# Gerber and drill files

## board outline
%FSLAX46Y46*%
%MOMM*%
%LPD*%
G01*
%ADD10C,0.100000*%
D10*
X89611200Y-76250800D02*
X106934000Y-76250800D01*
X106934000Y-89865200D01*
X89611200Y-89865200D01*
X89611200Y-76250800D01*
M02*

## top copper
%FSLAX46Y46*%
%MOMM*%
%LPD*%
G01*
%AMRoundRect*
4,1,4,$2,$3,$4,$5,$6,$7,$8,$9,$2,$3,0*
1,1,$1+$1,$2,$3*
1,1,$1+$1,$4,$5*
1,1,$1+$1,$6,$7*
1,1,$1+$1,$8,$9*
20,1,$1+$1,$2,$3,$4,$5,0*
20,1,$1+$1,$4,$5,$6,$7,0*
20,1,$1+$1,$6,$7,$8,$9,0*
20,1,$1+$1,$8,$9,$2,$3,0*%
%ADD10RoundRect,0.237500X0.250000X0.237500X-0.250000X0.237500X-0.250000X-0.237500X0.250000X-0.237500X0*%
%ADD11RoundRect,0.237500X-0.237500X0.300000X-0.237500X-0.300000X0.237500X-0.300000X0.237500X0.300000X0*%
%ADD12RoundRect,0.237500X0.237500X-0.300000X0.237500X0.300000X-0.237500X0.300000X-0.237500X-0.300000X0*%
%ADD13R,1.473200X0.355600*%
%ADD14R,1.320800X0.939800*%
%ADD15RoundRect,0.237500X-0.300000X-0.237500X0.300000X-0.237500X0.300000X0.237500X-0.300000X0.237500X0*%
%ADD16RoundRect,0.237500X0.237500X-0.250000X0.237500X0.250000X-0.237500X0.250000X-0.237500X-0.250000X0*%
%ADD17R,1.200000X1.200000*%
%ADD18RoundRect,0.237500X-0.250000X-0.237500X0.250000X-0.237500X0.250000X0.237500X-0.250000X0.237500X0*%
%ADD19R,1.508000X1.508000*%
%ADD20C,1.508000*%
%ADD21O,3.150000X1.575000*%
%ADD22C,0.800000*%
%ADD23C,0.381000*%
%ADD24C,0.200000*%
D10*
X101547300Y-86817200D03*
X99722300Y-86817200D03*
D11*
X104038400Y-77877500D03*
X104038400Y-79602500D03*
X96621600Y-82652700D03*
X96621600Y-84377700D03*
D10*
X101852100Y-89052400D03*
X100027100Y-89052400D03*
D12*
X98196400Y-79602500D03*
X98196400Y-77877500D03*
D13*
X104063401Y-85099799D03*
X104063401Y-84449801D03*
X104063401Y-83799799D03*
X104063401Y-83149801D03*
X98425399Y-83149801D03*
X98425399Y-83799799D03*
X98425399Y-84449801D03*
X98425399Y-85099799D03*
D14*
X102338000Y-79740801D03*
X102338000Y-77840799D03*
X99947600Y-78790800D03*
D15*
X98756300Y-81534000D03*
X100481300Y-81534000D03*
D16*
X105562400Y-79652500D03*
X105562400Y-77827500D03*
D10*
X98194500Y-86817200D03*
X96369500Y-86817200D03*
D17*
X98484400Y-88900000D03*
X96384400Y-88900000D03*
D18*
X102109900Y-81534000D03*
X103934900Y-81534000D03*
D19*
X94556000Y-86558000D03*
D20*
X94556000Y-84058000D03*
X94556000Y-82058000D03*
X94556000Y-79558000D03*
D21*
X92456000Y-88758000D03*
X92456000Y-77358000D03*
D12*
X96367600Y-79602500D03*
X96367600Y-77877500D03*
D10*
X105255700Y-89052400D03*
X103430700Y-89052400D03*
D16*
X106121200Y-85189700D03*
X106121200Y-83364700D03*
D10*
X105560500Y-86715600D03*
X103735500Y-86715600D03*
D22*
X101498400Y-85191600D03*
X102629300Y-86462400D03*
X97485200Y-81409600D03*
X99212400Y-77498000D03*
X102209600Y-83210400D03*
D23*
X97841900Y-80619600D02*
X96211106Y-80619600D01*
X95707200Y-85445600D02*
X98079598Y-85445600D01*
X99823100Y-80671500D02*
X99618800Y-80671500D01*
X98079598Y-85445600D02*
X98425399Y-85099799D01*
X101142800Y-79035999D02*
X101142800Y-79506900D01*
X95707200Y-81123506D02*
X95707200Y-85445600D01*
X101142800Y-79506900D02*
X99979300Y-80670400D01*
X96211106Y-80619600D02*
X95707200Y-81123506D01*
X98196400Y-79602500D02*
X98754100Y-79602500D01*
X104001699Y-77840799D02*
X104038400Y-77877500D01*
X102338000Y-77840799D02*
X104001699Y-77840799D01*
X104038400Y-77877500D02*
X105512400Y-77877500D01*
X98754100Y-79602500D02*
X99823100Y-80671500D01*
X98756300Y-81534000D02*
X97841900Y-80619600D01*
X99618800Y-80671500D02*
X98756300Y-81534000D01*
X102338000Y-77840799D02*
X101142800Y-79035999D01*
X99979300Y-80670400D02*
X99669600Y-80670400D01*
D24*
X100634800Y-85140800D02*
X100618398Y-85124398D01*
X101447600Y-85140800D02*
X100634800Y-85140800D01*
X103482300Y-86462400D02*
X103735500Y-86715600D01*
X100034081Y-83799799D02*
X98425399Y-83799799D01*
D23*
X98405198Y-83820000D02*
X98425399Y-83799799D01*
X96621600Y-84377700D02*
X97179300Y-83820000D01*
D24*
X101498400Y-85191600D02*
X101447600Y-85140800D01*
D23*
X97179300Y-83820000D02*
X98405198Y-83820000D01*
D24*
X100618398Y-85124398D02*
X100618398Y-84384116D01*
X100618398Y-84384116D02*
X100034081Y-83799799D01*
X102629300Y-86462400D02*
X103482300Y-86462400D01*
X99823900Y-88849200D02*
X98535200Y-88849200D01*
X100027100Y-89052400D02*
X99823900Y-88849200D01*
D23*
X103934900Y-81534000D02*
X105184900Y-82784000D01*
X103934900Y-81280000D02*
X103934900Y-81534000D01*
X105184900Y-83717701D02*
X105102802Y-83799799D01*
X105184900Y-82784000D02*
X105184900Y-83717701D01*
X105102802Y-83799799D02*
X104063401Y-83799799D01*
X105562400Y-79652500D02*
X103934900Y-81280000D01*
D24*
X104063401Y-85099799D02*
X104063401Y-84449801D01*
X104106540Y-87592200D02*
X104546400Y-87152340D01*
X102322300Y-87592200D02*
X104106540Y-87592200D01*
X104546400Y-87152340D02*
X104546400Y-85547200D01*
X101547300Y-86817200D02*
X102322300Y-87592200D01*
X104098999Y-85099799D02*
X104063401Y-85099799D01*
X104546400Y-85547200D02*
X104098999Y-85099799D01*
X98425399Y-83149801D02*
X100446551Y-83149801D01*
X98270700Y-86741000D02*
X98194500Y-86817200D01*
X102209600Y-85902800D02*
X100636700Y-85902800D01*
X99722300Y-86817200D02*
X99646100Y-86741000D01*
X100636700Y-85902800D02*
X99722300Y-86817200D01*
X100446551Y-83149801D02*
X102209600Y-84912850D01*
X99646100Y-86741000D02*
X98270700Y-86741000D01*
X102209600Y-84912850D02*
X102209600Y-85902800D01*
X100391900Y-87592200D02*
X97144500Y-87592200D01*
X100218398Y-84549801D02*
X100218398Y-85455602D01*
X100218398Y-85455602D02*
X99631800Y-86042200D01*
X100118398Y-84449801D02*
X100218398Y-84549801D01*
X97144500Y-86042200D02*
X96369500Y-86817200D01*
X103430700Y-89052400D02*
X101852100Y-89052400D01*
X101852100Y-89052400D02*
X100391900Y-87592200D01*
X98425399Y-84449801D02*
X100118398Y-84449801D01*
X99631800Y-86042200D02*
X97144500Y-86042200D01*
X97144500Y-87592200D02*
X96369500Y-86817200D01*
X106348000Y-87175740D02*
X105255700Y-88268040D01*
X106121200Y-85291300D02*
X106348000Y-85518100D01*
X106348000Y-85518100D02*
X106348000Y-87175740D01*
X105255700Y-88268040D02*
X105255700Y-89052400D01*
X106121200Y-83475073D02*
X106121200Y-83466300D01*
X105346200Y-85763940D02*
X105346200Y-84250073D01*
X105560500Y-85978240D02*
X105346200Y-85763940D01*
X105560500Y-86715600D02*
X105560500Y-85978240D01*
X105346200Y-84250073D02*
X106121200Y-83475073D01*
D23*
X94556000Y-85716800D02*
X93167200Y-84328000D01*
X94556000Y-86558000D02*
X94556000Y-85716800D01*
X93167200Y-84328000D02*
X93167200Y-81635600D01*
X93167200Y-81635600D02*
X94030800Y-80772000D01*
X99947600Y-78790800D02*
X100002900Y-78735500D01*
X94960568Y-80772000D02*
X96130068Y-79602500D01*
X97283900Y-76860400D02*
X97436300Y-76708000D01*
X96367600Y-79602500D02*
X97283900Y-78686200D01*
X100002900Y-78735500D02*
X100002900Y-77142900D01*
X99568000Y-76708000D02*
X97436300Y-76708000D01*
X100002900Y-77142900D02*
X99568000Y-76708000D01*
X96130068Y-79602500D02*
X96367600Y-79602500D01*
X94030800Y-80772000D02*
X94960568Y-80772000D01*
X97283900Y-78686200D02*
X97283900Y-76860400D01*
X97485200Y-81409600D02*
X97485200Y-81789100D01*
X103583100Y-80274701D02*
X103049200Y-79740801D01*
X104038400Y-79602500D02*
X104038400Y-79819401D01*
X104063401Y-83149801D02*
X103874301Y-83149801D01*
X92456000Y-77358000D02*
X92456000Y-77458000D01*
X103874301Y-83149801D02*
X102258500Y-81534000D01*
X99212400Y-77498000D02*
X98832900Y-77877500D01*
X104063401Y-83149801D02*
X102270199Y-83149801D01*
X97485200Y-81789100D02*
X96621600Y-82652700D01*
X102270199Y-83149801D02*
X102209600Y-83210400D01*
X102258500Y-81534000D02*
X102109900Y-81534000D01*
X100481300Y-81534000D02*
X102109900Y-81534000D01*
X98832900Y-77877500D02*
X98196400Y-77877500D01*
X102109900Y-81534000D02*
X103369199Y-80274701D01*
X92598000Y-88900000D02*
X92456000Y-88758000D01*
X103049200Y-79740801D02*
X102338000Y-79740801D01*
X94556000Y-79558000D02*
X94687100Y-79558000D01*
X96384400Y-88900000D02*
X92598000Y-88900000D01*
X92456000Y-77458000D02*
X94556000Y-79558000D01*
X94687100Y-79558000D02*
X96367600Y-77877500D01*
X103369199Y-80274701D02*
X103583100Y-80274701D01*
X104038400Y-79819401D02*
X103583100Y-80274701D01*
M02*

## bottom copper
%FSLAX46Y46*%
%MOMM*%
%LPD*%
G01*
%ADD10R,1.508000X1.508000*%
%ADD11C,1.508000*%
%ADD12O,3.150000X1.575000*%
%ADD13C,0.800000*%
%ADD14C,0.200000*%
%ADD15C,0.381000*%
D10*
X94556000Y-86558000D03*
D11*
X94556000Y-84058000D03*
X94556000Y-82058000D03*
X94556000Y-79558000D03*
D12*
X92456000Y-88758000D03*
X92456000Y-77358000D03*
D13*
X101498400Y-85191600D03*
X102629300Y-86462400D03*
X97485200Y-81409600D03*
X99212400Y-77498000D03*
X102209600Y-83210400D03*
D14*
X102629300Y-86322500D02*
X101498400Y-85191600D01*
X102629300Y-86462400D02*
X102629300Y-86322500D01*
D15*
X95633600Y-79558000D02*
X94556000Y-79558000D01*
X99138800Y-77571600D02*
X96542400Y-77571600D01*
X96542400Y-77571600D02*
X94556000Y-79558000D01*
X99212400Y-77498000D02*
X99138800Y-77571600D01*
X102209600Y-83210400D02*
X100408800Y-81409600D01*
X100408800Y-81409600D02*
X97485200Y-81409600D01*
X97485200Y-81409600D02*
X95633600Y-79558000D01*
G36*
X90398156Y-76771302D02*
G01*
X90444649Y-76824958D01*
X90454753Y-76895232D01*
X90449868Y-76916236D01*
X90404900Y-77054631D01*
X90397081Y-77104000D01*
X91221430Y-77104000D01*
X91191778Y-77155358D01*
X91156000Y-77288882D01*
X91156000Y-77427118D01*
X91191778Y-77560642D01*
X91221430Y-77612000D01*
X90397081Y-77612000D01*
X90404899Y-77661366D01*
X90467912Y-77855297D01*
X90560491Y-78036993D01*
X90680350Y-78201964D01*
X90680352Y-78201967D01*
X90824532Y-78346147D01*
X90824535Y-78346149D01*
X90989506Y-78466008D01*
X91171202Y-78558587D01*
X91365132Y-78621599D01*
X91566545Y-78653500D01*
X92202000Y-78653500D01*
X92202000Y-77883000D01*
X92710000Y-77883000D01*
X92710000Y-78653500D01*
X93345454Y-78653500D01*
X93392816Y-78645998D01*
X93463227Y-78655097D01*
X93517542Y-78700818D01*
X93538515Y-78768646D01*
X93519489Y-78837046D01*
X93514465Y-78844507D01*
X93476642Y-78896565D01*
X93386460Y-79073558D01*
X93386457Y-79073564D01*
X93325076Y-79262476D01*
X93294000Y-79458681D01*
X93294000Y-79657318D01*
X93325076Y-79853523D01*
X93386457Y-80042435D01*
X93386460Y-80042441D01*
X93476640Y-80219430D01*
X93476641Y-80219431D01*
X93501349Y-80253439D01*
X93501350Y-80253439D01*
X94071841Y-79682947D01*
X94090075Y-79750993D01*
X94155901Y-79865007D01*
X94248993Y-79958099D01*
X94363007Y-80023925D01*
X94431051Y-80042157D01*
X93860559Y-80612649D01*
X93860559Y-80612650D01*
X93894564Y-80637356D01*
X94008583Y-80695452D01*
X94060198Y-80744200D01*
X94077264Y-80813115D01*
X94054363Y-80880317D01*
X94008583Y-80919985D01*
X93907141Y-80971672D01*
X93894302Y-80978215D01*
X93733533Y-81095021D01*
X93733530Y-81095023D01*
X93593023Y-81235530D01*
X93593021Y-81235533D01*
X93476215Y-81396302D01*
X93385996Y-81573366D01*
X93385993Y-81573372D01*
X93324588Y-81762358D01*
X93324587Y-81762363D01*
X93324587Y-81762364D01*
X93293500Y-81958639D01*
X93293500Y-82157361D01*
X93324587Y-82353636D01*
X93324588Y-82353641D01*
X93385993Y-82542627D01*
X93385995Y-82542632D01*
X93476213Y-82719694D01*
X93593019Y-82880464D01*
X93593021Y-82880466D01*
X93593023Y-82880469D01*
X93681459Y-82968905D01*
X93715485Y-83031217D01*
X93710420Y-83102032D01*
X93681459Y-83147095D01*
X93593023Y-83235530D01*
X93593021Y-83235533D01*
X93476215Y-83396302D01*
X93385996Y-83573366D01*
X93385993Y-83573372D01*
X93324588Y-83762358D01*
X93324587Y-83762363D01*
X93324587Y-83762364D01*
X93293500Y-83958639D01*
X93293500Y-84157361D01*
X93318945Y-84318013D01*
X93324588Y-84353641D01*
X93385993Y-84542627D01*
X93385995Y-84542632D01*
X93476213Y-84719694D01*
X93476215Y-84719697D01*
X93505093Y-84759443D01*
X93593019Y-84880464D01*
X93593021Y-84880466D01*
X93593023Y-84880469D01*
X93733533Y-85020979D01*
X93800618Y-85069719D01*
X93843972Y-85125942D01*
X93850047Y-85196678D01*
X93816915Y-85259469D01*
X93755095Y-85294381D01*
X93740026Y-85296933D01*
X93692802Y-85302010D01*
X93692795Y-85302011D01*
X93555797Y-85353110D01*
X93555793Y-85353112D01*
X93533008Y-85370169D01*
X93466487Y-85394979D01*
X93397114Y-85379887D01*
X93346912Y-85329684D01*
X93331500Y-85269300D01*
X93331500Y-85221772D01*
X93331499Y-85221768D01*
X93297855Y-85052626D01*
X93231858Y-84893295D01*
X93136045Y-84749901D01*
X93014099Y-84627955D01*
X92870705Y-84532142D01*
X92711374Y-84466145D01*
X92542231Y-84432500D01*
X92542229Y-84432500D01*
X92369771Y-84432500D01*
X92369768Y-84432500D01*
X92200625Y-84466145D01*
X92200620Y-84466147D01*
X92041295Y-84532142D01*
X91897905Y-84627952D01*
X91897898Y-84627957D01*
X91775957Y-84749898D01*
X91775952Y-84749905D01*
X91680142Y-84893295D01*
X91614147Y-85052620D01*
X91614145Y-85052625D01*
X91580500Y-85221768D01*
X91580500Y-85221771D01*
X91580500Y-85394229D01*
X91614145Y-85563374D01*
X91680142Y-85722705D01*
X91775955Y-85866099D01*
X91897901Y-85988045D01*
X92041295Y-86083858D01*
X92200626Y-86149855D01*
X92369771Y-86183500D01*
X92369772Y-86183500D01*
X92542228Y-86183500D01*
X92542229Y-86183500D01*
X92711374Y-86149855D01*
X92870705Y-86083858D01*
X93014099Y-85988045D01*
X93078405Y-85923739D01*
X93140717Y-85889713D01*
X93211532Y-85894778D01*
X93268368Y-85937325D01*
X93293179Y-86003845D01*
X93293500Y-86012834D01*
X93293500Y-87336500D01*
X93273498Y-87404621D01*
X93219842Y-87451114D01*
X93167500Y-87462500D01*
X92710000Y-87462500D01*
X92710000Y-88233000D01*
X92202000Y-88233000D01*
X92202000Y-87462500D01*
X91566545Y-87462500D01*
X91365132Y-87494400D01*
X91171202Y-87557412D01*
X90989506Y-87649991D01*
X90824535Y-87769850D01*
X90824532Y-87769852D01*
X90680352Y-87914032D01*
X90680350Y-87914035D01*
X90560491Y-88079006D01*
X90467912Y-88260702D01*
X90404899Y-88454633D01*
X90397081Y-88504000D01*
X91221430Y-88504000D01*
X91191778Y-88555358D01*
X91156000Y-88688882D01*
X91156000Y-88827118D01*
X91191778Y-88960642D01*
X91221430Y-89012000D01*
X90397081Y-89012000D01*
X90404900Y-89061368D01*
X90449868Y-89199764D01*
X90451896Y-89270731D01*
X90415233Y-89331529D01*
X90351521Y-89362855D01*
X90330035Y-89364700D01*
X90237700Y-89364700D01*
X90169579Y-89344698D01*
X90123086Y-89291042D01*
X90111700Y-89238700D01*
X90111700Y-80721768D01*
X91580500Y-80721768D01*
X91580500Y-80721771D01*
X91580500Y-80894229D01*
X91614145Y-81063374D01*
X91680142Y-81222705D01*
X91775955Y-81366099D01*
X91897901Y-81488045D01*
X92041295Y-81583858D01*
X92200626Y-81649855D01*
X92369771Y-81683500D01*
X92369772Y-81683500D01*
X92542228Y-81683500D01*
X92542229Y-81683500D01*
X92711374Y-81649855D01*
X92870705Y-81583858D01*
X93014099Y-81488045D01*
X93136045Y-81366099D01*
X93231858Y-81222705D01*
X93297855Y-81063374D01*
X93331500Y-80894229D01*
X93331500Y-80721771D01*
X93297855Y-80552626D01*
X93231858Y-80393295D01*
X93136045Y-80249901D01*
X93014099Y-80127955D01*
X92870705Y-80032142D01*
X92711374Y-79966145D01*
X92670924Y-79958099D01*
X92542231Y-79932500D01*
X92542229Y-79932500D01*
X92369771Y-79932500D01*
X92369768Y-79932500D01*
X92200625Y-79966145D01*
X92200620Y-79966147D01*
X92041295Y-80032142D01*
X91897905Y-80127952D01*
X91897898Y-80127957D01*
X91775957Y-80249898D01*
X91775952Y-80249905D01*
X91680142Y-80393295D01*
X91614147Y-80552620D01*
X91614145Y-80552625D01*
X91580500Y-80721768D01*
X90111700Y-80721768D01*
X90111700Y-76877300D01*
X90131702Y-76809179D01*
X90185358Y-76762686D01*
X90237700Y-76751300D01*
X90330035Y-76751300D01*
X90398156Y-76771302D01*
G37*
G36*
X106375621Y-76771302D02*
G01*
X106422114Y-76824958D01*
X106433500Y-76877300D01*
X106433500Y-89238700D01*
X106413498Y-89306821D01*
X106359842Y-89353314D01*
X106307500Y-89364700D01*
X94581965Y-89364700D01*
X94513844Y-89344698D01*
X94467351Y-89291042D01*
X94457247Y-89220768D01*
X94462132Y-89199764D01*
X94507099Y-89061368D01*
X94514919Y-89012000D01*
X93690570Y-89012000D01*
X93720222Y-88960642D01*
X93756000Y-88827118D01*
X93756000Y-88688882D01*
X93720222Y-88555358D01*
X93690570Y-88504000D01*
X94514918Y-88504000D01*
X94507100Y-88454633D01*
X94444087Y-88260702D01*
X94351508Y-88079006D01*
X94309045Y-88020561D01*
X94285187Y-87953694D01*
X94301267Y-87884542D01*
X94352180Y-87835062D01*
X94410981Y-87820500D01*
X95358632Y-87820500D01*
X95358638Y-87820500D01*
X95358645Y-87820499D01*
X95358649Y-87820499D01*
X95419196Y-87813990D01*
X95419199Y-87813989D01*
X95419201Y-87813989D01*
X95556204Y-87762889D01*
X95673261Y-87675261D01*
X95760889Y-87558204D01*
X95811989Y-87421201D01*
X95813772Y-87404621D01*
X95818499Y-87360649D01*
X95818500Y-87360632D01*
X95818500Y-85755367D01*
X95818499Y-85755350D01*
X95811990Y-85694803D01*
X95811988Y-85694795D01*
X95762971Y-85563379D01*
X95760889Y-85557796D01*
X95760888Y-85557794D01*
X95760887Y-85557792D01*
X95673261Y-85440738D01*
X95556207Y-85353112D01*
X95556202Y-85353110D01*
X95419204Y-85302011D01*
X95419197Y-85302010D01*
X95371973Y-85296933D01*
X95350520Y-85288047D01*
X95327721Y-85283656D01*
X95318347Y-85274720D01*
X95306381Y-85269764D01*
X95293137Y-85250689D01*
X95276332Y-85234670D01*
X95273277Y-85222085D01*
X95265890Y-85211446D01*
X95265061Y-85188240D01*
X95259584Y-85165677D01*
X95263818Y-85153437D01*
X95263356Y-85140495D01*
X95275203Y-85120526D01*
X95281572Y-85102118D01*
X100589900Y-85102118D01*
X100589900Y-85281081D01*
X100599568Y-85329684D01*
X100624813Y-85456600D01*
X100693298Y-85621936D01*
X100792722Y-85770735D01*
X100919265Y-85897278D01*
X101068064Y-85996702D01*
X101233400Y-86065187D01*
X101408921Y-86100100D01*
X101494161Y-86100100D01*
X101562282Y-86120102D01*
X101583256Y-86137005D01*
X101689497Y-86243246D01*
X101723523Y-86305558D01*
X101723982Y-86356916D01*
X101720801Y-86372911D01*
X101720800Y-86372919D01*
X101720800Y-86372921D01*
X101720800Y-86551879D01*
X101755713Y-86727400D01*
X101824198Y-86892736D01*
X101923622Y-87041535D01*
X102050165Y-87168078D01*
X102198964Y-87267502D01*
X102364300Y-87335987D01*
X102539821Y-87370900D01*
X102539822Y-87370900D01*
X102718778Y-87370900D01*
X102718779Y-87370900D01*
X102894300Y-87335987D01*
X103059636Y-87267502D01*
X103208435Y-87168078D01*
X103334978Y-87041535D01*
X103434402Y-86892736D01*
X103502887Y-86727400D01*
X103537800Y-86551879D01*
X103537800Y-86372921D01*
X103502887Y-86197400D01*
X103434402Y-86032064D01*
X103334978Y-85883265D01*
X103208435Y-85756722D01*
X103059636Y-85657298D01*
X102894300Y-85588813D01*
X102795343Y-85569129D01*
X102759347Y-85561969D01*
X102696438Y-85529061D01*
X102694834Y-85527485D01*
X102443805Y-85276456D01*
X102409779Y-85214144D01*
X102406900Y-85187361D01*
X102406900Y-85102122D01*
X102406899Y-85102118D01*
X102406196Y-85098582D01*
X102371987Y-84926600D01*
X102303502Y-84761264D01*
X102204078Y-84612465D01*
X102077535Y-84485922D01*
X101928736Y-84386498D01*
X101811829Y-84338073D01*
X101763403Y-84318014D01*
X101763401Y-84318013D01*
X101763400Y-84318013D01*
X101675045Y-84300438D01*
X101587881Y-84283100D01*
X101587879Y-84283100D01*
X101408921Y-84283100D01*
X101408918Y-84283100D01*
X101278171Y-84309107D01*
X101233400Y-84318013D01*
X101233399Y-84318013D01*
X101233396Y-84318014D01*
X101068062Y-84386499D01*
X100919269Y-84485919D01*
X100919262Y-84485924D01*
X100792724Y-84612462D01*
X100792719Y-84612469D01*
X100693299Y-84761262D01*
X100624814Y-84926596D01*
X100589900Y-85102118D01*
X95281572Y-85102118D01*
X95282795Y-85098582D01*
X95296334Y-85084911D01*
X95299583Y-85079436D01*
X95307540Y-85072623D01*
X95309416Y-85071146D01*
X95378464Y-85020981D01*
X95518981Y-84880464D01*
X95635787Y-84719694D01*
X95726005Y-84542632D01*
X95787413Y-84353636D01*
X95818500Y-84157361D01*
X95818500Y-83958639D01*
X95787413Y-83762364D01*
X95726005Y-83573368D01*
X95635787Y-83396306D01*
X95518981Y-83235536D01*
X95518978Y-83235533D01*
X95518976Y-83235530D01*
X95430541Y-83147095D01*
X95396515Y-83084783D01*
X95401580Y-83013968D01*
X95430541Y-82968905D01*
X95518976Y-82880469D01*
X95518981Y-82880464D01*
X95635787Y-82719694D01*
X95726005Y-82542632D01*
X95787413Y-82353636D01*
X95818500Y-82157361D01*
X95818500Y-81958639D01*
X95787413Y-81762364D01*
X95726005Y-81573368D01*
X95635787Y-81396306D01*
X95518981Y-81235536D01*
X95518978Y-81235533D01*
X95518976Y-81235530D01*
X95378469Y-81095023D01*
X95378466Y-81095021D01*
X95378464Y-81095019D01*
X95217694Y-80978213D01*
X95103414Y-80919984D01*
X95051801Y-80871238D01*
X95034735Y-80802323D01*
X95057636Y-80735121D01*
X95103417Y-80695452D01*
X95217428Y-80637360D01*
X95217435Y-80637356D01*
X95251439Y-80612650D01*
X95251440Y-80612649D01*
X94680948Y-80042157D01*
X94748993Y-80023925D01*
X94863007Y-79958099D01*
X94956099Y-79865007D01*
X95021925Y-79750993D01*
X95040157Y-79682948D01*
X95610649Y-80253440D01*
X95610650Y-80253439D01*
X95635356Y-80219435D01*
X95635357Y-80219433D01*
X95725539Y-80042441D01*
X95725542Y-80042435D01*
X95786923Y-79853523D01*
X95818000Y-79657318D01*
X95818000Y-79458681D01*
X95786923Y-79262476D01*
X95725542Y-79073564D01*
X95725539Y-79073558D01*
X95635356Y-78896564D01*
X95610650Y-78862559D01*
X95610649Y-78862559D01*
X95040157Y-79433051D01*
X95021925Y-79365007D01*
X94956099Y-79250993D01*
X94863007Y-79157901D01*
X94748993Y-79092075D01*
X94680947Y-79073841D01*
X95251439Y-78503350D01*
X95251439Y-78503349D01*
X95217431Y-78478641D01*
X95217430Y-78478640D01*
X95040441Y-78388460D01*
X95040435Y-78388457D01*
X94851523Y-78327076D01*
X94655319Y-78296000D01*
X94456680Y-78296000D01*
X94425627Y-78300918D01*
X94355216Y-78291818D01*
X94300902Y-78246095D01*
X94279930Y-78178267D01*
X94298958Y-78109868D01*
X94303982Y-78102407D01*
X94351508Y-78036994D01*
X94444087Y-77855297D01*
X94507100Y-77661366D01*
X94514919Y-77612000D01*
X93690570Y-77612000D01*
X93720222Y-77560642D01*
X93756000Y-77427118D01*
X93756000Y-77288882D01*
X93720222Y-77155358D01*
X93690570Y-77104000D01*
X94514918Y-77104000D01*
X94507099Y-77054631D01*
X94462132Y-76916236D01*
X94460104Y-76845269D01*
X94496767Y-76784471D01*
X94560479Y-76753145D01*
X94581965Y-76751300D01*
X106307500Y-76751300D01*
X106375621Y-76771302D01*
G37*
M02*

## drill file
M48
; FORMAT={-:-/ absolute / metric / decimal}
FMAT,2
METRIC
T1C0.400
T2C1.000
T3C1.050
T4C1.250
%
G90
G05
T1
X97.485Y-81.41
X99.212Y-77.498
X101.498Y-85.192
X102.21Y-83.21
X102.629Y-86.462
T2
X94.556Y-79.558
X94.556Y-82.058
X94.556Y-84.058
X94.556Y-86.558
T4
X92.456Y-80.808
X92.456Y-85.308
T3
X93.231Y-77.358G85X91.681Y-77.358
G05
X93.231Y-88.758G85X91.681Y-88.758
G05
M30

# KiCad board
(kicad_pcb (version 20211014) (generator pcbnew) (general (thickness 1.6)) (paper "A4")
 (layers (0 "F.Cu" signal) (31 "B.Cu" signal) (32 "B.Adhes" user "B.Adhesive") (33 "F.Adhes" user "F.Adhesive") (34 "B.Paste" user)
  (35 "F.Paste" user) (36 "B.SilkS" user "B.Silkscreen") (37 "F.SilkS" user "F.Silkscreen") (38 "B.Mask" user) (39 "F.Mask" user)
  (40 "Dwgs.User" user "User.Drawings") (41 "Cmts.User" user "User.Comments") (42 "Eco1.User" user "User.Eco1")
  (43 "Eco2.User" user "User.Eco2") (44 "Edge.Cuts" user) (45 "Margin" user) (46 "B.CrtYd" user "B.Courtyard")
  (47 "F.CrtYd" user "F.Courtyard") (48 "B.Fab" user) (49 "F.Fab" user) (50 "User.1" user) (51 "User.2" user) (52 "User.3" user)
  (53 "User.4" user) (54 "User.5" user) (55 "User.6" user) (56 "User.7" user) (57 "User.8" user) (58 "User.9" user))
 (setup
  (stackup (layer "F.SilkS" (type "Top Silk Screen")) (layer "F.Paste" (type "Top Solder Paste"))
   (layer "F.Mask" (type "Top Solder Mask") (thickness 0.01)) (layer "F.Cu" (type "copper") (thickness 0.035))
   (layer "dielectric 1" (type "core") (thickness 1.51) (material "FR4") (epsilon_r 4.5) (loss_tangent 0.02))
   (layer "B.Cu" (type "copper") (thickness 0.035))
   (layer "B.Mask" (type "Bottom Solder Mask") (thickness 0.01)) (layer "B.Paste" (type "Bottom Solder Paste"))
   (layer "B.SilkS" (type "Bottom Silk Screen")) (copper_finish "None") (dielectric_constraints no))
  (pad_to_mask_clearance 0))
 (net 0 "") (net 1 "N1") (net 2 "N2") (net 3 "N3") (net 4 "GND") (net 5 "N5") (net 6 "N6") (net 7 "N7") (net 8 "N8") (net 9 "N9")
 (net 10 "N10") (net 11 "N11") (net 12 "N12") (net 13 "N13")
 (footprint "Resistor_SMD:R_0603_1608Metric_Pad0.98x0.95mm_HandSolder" (layer "F.Cu") (at 100.6348 86.8172 180)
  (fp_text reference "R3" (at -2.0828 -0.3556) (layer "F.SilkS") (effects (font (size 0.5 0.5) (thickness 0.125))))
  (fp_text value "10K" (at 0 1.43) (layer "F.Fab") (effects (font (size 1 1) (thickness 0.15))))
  (pad "1" smd roundrect (at -0.9125 0 180) (size 0.975 0.95) (layers "F.Cu" "F.Paste" "F.Mask") (roundrect_rratio 0.25) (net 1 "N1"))
  (pad "2" smd roundrect (at 0.9125 0 180) (size 0.975 0.95) (layers "F.Cu" "F.Paste" "F.Mask") (roundrect_rratio 0.25) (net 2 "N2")))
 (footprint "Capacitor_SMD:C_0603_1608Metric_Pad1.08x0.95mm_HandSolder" (layer "F.Cu") (at 104.0384 78.74 -90)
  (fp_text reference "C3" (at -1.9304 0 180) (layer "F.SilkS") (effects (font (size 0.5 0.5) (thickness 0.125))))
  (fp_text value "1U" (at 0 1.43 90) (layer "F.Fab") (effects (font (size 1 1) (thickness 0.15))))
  (pad "1" smd roundrect (at -0.8625 0 270) (size 1.075 0.95) (layers "F.Cu" "F.Paste" "F.Mask") (roundrect_rratio 0.25) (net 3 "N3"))
  (pad "2" smd roundrect (at 0.8625 0 270) (size 1.075 0.95) (layers "F.Cu" "F.Paste" "F.Mask") (roundrect_rratio 0.25) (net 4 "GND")))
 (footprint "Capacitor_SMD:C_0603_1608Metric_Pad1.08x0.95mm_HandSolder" (layer "F.Cu") (at 96.6216 83.5152 -90)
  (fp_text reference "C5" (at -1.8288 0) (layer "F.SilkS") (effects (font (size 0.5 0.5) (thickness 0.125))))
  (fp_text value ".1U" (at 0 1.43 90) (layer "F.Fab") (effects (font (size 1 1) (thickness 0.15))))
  (pad "1" smd roundrect (at -0.8625 0 270) (size 1.075 0.95) (layers "F.Cu" "F.Paste" "F.Mask") (roundrect_rratio 0.25) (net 4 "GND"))
  (pad "2" smd roundrect (at 0.8625 0 270) (size 1.075 0.95) (layers "F.Cu" "F.Paste" "F.Mask") (roundrect_rratio 0.25) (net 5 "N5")))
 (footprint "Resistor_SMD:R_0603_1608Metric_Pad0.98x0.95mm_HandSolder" (layer "F.Cu") (at 100.9396 89.0524 180)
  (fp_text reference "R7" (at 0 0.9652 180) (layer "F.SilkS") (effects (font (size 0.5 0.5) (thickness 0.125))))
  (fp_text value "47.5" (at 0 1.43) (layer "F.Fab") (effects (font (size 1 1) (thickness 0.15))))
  (pad "1" smd roundrect (at -0.9125 0 180) (size 0.975 0.95) (layers "F.Cu" "F.Paste" "F.Mask") (roundrect_rratio 0.25) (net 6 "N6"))
  (pad "2" smd roundrect (at 0.9125 0 180) (size 0.975 0.95) (layers "F.Cu" "F.Paste" "F.Mask") (roundrect_rratio 0.25) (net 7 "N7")))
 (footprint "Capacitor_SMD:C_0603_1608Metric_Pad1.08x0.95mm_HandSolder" (layer "F.Cu") (at 98.1964 78.74 90)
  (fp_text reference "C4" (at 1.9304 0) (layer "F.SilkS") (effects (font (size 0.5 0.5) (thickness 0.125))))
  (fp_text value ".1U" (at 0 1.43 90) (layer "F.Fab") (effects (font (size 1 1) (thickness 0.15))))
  (pad "1" smd roundrect (at -0.8625 0 90) (size 1.075 0.95) (layers "F.Cu" "F.Paste" "F.Mask") (roundrect_rratio 0.25) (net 3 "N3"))
  (pad "2" smd roundrect (at 0.8625 0 90) (size 1.075 0.95) (layers "F.Cu" "F.Paste" "F.Mask") (roundrect_rratio 0.25) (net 4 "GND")))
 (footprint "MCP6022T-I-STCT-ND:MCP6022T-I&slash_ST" (layer "F.Cu") (at 101.2444 84.1248 180)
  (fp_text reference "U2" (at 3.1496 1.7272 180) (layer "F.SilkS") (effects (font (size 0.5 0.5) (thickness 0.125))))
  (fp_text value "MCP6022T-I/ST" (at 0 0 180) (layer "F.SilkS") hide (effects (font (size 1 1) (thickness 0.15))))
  (pad "1" smd rect locked (at -2.819001 -0.974999 180) (size 1.4732 0.3556) (layers "F.Cu" "F.Paste" "F.Mask") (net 1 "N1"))
  (pad "2" smd rect locked (at -2.819001 -0.325001 180) (size 1.4732 0.3556) (layers "F.Cu" "F.Paste" "F.Mask") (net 1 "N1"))
  (pad "3" smd rect locked (at -2.819001 0.325001 180) (size 1.4732 0.3556) (layers "F.Cu" "F.Paste" "F.Mask") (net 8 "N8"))
  (pad "4" smd rect locked (at -2.819001 0.974999 180) (size 1.4732 0.3556) (layers "F.Cu" "F.Paste" "F.Mask") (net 4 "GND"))
  (pad "5" smd rect locked (at 2.819001 0.974999 180) (size 1.4732 0.3556) (layers "F.Cu" "F.Paste" "F.Mask") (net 2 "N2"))
  (pad "6" smd rect locked (at 2.819001 0.325001 180) (size 1.4732 0.3556) (layers "F.Cu" "F.Paste" "F.Mask") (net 5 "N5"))
  (pad "7" smd rect locked (at 2.819001 -0.325001 180) (size 1.4732 0.3556) (layers "F.Cu" "F.Paste" "F.Mask") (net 6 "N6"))
  (pad "8" smd rect locked (at 2.819001 -0.974999 180) (size 1.4732 0.3556) (layers "F.Cu" "F.Paste" "F.Mask") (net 3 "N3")))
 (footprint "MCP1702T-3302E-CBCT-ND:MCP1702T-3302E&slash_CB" (layer "F.Cu") (at 101.1428 78.7908 90)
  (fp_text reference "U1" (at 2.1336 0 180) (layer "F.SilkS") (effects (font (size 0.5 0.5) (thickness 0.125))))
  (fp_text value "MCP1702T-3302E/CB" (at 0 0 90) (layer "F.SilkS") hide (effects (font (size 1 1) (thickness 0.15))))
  (pad "1" smd rect locked (at -0.950001 1.1952 90) (size 0.9398 1.3208) (layers "F.Cu" "F.Paste" "F.Mask") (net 4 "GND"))
  (pad "2" smd rect locked (at 0.950001 1.1952 90) (size 0.9398 1.3208) (layers "F.Cu" "F.Paste" "F.Mask") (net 3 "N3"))
  (pad "3" smd rect locked (at 0 -1.1952 90) (size 0.9398 1.3208) (layers "F.Cu" "F.Paste" "F.Mask") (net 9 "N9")))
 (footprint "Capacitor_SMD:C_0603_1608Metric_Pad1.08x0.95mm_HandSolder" (layer "F.Cu") (at 99.6188 81.534)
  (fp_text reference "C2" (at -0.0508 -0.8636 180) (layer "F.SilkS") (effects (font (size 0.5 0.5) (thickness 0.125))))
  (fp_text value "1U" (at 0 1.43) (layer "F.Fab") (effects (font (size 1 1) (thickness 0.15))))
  (pad "1" smd roundrect (at -0.8625 0) (size 1.075 0.95) (layers "F.Cu" "F.Paste" "F.Mask") (roundrect_rratio 0.25) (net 3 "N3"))
  (pad "2" smd roundrect (at 0.8625 0) (size 1.075 0.95) (layers "F.Cu" "F.Paste" "F.Mask") (roundrect_rratio 0.25) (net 4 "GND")))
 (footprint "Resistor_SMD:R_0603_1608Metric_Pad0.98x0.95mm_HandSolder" (layer "F.Cu") (at 105.5624 78.74 90)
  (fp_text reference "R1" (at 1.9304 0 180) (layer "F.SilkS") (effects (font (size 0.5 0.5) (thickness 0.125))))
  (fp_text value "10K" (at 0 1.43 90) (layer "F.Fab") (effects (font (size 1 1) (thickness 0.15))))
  (pad "1" smd roundrect (at -0.9125 0 90) (size 0.975 0.95) (layers "F.Cu" "F.Paste" "F.Mask") (roundrect_rratio 0.25) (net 8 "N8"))
  (pad "2" smd roundrect (at 0.9125 0 90) (size 0.975 0.95) (layers "F.Cu" "F.Paste" "F.Mask") (roundrect_rratio 0.25) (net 3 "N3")))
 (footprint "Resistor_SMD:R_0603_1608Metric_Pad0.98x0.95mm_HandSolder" (layer "F.Cu") (at 97.282 86.8172 180)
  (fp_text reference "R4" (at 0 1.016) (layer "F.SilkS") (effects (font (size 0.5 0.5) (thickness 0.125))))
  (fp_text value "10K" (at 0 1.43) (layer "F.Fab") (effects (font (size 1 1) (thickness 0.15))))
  (pad "1" smd roundrect (at -0.9125 0 180) (size 0.975 0.95) (layers "F.Cu" "F.Paste" "F.Mask") (roundrect_rratio 0.25) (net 2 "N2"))
  (pad "2" smd roundrect (at 0.9125 0 180) (size 0.975 0.95) (layers "F.Cu" "F.Paste" "F.Mask") (roundrect_rratio 0.25) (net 6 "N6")))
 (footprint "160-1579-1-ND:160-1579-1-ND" (layer "F.Cu") (at 97.4344 88.9)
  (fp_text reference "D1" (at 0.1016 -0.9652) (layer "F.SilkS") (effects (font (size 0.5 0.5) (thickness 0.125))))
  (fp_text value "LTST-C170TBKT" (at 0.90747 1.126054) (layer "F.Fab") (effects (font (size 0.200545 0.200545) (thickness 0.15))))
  (pad "+" smd rect locked (at 1.05 0) (size 1.2 1.2) (layers "F.Cu" "F.Paste" "F.Mask") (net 7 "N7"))
  (pad "-" smd rect locked (at -1.05 0) (size 1.2 1.2) (layers "F.Cu" "F.Paste" "F.Mask") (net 4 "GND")))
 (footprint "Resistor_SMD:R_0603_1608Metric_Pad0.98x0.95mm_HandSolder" (layer "F.Cu") (at 103.0224 81.534)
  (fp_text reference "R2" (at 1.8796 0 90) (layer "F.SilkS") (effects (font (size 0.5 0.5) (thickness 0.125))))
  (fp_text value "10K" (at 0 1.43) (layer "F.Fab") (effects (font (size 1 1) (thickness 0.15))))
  (pad "1" smd roundrect (at -0.9125 0) (size 0.975 0.95) (layers "F.Cu" "F.Paste" "F.Mask") (roundrect_rratio 0.25) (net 4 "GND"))
  (pad "2" smd roundrect (at 0.9125 0) (size 0.975 0.95) (layers "F.Cu" "F.Paste" "F.Mask") (roundrect_rratio 0.25) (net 8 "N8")))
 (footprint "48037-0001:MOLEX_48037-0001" (layer "F.Cu") (at 92.456 83.058 -90)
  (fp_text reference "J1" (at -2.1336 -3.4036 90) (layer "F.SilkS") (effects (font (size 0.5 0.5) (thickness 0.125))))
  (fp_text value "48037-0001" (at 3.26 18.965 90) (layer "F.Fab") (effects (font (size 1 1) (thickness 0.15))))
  (pad "" np_thru_hole circle (at -2.25 0 270) (size 1.25 1.25) (drill 1.25) (layers *.Cu *.Mask))
  (pad "" np_thru_hole circle (at 2.25 0 270) (size 1.25 1.25) (drill 1.25) (layers *.Cu *.Mask))
  (pad "1" thru_hole rect (at 3.5 -2.1 270) (size 1.508 1.508) (drill 1) (layers *.Cu *.Mask) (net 9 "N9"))
  (pad "2" thru_hole circle (at 1 -2.1 270) (size 1.508 1.508) (drill 1) (layers *.Cu *.Mask) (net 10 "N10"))
  (pad "3" thru_hole circle (at -1 -2.1 270) (size 1.508 1.508) (drill 1) (layers *.Cu *.Mask) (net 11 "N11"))
  (pad "4" thru_hole circle (at -3.5 -2.1 270) (size 1.508 1.508) (drill 1) (layers *.Cu *.Mask) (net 4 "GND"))
  (pad "S1" thru_hole oval (at 5.7 0 270) (size 1.575 3.15) (drill oval 1.05 2.6) (layers *.Cu *.Mask) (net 4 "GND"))
  (pad "S2" thru_hole oval (at -5.7 0 270) (size 1.575 3.15) (drill oval 1.05 2.6) (layers *.Cu *.Mask) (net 4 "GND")))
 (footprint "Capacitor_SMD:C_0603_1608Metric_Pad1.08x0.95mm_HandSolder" (layer "F.Cu") (at 96.3676 78.74 90)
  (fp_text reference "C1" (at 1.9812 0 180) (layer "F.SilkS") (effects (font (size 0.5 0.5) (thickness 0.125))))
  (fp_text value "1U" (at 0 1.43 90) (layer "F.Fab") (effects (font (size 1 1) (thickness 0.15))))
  (pad "1" smd roundrect (at -0.8625 0 90) (size 1.075 0.95) (layers "F.Cu" "F.Paste" "F.Mask") (roundrect_rratio 0.25) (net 9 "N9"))
  (pad "2" smd roundrect (at 0.8625 0 90) (size 1.075 0.95) (layers "F.Cu" "F.Paste" "F.Mask") (roundrect_rratio 0.25) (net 4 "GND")))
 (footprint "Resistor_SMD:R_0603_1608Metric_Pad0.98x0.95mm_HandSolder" (layer "F.Cu") (at 104.3432 89.0524 180)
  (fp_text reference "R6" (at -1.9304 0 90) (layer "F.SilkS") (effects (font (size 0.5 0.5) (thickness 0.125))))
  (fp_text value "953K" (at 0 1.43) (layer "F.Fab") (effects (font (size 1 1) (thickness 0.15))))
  (pad "1" smd roundrect (at -0.9125 0 180) (size 0.975 0.95) (layers "F.Cu" "F.Paste" "F.Mask") (roundrect_rratio 0.25) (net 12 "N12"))
  (pad "2" smd roundrect (at 0.9125 0 180) (size 0.975 0.95) (layers "F.Cu" "F.Paste" "F.Mask") (roundrect_rratio 0.25) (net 6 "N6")))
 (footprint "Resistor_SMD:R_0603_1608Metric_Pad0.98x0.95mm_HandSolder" (layer "F.Cu") (at 106.1212 84.2772 90)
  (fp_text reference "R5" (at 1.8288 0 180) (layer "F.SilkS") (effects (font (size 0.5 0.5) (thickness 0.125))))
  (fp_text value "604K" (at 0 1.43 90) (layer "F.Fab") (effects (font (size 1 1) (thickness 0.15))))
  (pad "1" smd roundrect (at -0.9125 0 90) (size 0.975 0.95) (layers "F.Cu" "F.Paste" "F.Mask") (roundrect_rratio 0.25) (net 12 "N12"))
  (pad "2" smd roundrect (at 0.9125 0 90) (size 0.975 0.95) (layers "F.Cu" "F.Paste" "F.Mask") (roundrect_rratio 0.25) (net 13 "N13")))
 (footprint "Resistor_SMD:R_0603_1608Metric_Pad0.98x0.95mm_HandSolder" (layer "F.Cu") (at 104.648 86.7156 180)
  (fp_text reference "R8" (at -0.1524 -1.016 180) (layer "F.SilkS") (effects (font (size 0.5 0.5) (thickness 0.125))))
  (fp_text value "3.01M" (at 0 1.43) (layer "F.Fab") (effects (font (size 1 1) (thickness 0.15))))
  (pad "1" smd roundrect (at -0.9125 0 180) (size 0.975 0.95) (layers "F.Cu" "F.Paste" "F.Mask") (roundrect_rratio 0.25) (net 13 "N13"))
  (pad "2" smd roundrect (at 0.9125 0 180) (size 0.975 0.95) (layers "F.Cu" "F.Paste" "F.Mask") (roundrect_rratio 0.25) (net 5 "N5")))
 (gr_rect (start 89.6112 76.2508) (end 106.934 89.8652) (layer "Edge.Cuts") (width 0.1) (fill none))
 (segment (start 97.8419 80.6196) (end 96.211106 80.6196) (width 0.381) (layer "F.Cu") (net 3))
 (segment (start 95.7072 85.4456) (end 98.079598 85.4456) (width 0.381) (layer "F.Cu") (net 3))
 (segment (start 99.8231 80.6715) (end 99.6188 80.6715) (width 0.381) (layer "F.Cu") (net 3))
 (segment (start 98.079598 85.4456) (end 98.425399 85.099799) (width 0.381) (layer "F.Cu") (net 3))
 (segment (start 101.1428 79.035999) (end 101.1428 79.5069) (width 0.381) (layer "F.Cu") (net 3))
 (segment (start 95.7072 81.123506) (end 95.7072 85.4456) (width 0.381) (layer "F.Cu") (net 3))
 (segment (start 101.1428 79.5069) (end 99.9793 80.6704) (width 0.381) (layer "F.Cu") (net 3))
 (segment (start 96.211106 80.6196) (end 95.7072 81.123506) (width 0.381) (layer "F.Cu") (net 3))
 (segment (start 98.1964 79.6025) (end 98.7541 79.6025) (width 0.381) (layer "F.Cu") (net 3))
 (segment (start 104.001699 77.840799) (end 104.0384 77.8775) (width 0.381) (layer "F.Cu") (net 3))
 (segment (start 102.338 77.840799) (end 104.001699 77.840799) (width 0.381) (layer "F.Cu") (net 3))
 (segment (start 104.0384 77.8775) (end 105.5124 77.8775) (width 0.381) (layer "F.Cu") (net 3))
 (segment (start 98.7541 79.6025) (end 99.8231 80.6715) (width 0.381) (layer "F.Cu") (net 3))
 (segment (start 98.7563 81.534) (end 97.8419 80.6196) (width 0.381) (layer "F.Cu") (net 3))
 (segment (start 99.6188 80.6715) (end 98.7563 81.534) (width 0.381) (layer "F.Cu") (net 3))
 (segment (start 102.338 77.840799) (end 101.1428 79.035999) (width 0.381) (layer "F.Cu") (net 3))
 (segment (start 99.9793 80.6704) (end 99.6696 80.6704) (width 0.381) (layer "F.Cu") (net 3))
 (segment (start 100.6348 85.1408) (end 100.618398 85.124398) (width 0.2) (layer "F.Cu") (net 5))
 (segment (start 101.4476 85.1408) (end 100.6348 85.1408) (width 0.2) (layer "F.Cu") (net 5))
 (segment (start 103.4823 86.4624) (end 103.7355 86.7156) (width 0.2) (layer "F.Cu") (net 5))
 (segment (start 100.034081 83.799799) (end 98.425399 83.799799) (width 0.2) (layer "F.Cu") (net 5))
 (segment (start 98.405198 83.82) (end 98.425399 83.799799) (width 0.381) (layer "F.Cu") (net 5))
 (segment (start 96.6216 84.3777) (end 97.1793 83.82) (width 0.381) (layer "F.Cu") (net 5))
 (segment (start 101.4984 85.1916) (end 101.4476 85.1408) (width 0.2) (layer "F.Cu") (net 5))
 (segment (start 97.1793 83.82) (end 98.405198 83.82) (width 0.381) (layer "F.Cu") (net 5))
 (segment (start 100.618398 85.124398) (end 100.618398 84.384116) (width 0.2) (layer "F.Cu") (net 5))
 (segment (start 100.618398 84.384116) (end 100.034081 83.799799) (width 0.2) (layer "F.Cu") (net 5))
 (segment (start 102.6293 86.4624) (end 103.4823 86.4624) (width 0.2) (layer "F.Cu") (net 5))
 (via (at 101.4984 85.1916) (size 0.8) (drill 0.4) (layers "F.Cu" "B.Cu") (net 5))
 (via (at 102.6293 86.4624) (size 0.8) (drill 0.4) (layers "F.Cu" "B.Cu") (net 5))
 (segment (start 102.6293 86.3225) (end 101.4984 85.1916) (width 0.2) (layer "B.Cu") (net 5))
 (segment (start 102.6293 86.4624) (end 102.6293 86.3225) (width 0.2) (layer "B.Cu") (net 5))
 (segment (start 99.8239 88.8492) (end 98.5352 88.8492) (width 0.2) (layer "F.Cu") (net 7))
 (segment (start 100.0271 89.0524) (end 99.8239 88.8492) (width 0.2) (layer "F.Cu") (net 7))
 (segment (start 103.9349 81.534) (end 105.1849 82.784) (width 0.381) (layer "F.Cu") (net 8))
 (segment (start 103.9349 81.28) (end 103.9349 81.534) (width 0.381) (layer "F.Cu") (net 8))
 (segment (start 105.1849 83.717701) (end 105.102802 83.799799) (width 0.381) (layer "F.Cu") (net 8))
 (segment (start 105.1849 82.784) (end 105.1849 83.717701) (width 0.381) (layer "F.Cu") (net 8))
 (segment (start 105.102802 83.799799) (end 104.063401 83.799799) (width 0.381) (layer "F.Cu") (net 8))
 (segment (start 105.5624 79.6525) (end 103.9349 81.28) (width 0.381) (layer "F.Cu") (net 8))
 (segment (start 104.063401 85.099799) (end 104.063401 84.449801) (width 0.2) (layer "F.Cu") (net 1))
 (segment (start 104.10654 87.5922) (end 104.5464 87.15234) (width 0.2) (layer "F.Cu") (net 1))
 (segment (start 102.3223 87.5922) (end 104.10654 87.5922) (width 0.2) (layer "F.Cu") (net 1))
 (segment (start 104.5464 87.15234) (end 104.5464 85.5472) (width 0.2) (layer "F.Cu") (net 1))
 (segment (start 101.5473 86.8172) (end 102.3223 87.5922) (width 0.2) (layer "F.Cu") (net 1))
 (segment (start 104.098999 85.099799) (end 104.063401 85.099799) (width 0.2) (layer "F.Cu") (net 1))
 (segment (start 104.5464 85.5472) (end 104.098999 85.099799) (width 0.2) (layer "F.Cu") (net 1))
 (segment (start 98.425399 83.149801) (end 100.446551 83.149801) (width 0.2) (layer "F.Cu") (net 2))
 (segment (start 98.2707 86.741) (end 98.1945 86.8172) (width 0.2) (layer "F.Cu") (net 2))
 (segment (start 102.2096 85.9028) (end 100.6367 85.9028) (width 0.2) (layer "F.Cu") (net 2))
 (segment (start 99.7223 86.8172) (end 99.6461 86.741) (width 0.2) (layer "F.Cu") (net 2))
 (segment (start 100.6367 85.9028) (end 99.7223 86.8172) (width 0.2) (layer "F.Cu") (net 2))
 (segment (start 100.446551 83.149801) (end 102.2096 84.91285) (width 0.2) (layer "F.Cu") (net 2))
 (segment (start 99.6461 86.741) (end 98.2707 86.741) (width 0.2) (layer "F.Cu") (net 2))
 (segment (start 102.2096 84.91285) (end 102.2096 85.9028) (width 0.2) (layer "F.Cu") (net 2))
 (segment (start 100.3919 87.5922) (end 97.1445 87.5922) (width 0.2) (layer "F.Cu") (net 6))
 (segment (start 100.218398 84.549801) (end 100.218398 85.455602) (width 0.2) (layer "F.Cu") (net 6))
 (segment (start 100.218398 85.455602) (end 99.6318 86.0422) (width 0.2) (layer "F.Cu") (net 6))
 (segment (start 100.118398 84.449801) (end 100.218398 84.549801) (width 0.2) (layer "F.Cu") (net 6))
 (segment (start 97.1445 86.0422) (end 96.3695 86.8172) (width 0.2) (layer "F.Cu") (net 6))
 (segment (start 103.4307 89.0524) (end 101.8521 89.0524) (width 0.2) (layer "F.Cu") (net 6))
 (segment (start 101.8521 89.0524) (end 100.3919 87.5922) (width 0.2) (layer "F.Cu") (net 6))
 (segment (start 98.425399 84.449801) (end 100.118398 84.449801) (width 0.2) (layer "F.Cu") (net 6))
 (segment (start 99.6318 86.0422) (end 97.1445 86.0422) (width 0.2) (layer "F.Cu") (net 6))
 (segment (start 97.1445 87.5922) (end 96.3695 86.8172) (width 0.2) (layer "F.Cu") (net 6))
 (segment (start 106.348 87.17574) (end 105.2557 88.26804) (width 0.2) (layer "F.Cu") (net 12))
 (segment (start 106.1212 85.2913) (end 106.348 85.5181) (width 0.2) (layer "F.Cu") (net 12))
 (segment (start 106.348 85.5181) (end 106.348 87.17574) (width 0.2) (layer "F.Cu") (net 12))
 (segment (start 105.2557 88.26804) (end 105.2557 89.0524) (width 0.2) (layer "F.Cu") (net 12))
 (segment (start 106.1212 83.475073) (end 106.1212 83.4663) (width 0.2) (layer "F.Cu") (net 13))
 (segment (start 105.3462 85.76394) (end 105.3462 84.250073) (width 0.2) (layer "F.Cu") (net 13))
 (segment (start 105.5605 85.97824) (end 105.3462 85.76394) (width 0.2) (layer "F.Cu") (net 13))
 (segment (start 105.5605 86.7156) (end 105.5605 85.97824) (width 0.2) (layer "F.Cu") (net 13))
 (segment (start 105.3462 84.250073) (end 106.1212 83.475073) (width 0.2) (layer "F.Cu") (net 13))
 (segment (start 94.556 85.7168) (end 93.1672 84.328) (width 0.381) (layer "F.Cu") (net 9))
 (segment (start 94.556 86.558) (end 94.556 85.7168) (width 0.381) (layer "F.Cu") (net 9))
 (segment (start 93.1672 84.328) (end 93.1672 81.6356) (width 0.381) (layer "F.Cu") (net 9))
 (segment (start 93.1672 81.6356) (end 94.0308 80.772) (width 0.381) (layer "F.Cu") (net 9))
 (segment (start 99.9476 78.7908) (end 100.0029 78.7355) (width 0.381) (layer "F.Cu") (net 9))
 (segment (start 94.960568 80.772) (end 96.130068 79.6025) (width 0.381) (layer "F.Cu") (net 9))
 (segment (start 97.2839 76.8604) (end 97.4363 76.708) (width 0.381) (layer "F.Cu") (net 9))
 (segment (start 96.3676 79.6025) (end 97.2839 78.6862) (width 0.381) (layer "F.Cu") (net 9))
 (segment (start 100.0029 78.7355) (end 100.0029 77.1429) (width 0.381) (layer "F.Cu") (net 9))
 (segment (start 99.568 76.708) (end 97.4363 76.708) (width 0.381) (layer "F.Cu") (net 9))
 (segment (start 100.0029 77.1429) (end 99.568 76.708) (width 0.381) (layer "F.Cu") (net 9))
 (segment (start 96.130068 79.6025) (end 96.3676 79.6025) (width 0.381) (layer "F.Cu") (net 9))
 (segment (start 94.0308 80.772) (end 94.960568 80.772) (width 0.381) (layer "F.Cu") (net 9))
 (segment (start 97.2839 78.6862) (end 97.2839 76.8604) (width 0.381) (layer "F.Cu") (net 9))
 (segment (start 97.4852 81.4096) (end 97.4852 81.7891) (width 0.381) (layer "F.Cu") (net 4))
 (segment (start 103.5831 80.274701) (end 103.0492 79.740801) (width 0.381) (layer "F.Cu") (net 4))
 (segment (start 104.0384 79.6025) (end 104.0384 79.819401) (width 0.381) (layer "F.Cu") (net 4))
 (segment (start 104.063401 83.149801) (end 103.874301 83.149801) (width 0.381) (layer "F.Cu") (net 4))
 (segment (start 92.456 77.358) (end 92.456 77.458) (width 0.381) (layer "F.Cu") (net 4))
 (segment (start 103.874301 83.149801) (end 102.2585 81.534) (width 0.381) (layer "F.Cu") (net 4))
 (segment (start 99.2124 77.498) (end 98.8329 77.8775) (width 0.381) (layer "F.Cu") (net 4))
 (segment (start 104.063401 83.149801) (end 102.270199 83.149801) (width 0.381) (layer "F.Cu") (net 4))
 (segment (start 97.4852 81.7891) (end 96.6216 82.6527) (width 0.381) (layer "F.Cu") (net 4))
 (segment (start 102.270199 83.149801) (end 102.2096 83.2104) (width 0.381) (layer "F.Cu") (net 4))
 (segment (start 102.2585 81.534) (end 102.1099 81.534) (width 0.381) (layer "F.Cu") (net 4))
 (segment (start 100.4813 81.534) (end 102.1099 81.534) (width 0.381) (layer "F.Cu") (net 4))
 (segment (start 98.8329 77.8775) (end 98.1964 77.8775) (width 0.381) (layer "F.Cu") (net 4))
 (segment (start 102.1099 81.534) (end 103.369199 80.274701) (width 0.381) (layer "F.Cu") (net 4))
 (segment (start 92.598 88.9) (end 92.456 88.758) (width 0.381) (layer "F.Cu") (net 4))
 (segment (start 103.0492 79.740801) (end 102.338 79.740801) (width 0.381) (layer "F.Cu") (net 4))
 (segment (start 94.556 79.558) (end 94.6871 79.558) (width 0.381) (layer "F.Cu") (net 4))
 (segment (start 96.3844 88.9) (end 92.598 88.9) (width 0.381) (layer "F.Cu") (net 4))
 (segment (start 92.456 77.458) (end 94.556 79.558) (width 0.381) (layer "F.Cu") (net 4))
 (segment (start 94.6871 79.558) (end 96.3676 77.8775) (width 0.381) (layer "F.Cu") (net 4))
 (segment (start 103.369199 80.274701) (end 103.5831 80.274701) (width 0.381) (layer "F.Cu") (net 4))
 (segment (start 104.0384 79.819401) (end 103.5831 80.274701) (width 0.381) (layer "F.Cu") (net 4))
 (via (at 97.4852 81.4096) (size 0.8) (drill 0.4) (layers "F.Cu" "B.Cu") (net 4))
 (via (at 99.2124 77.498) (size 0.8) (drill 0.4) (layers "F.Cu" "B.Cu") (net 4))
 (via (at 102.2096 83.2104) (size 0.8) (drill 0.4) (layers "F.Cu" "B.Cu") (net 4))
 (segment (start 95.6336 79.558) (end 94.556 79.558) (width 0.381) (layer "B.Cu") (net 4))
 (segment (start 99.1388 77.5716) (end 96.5424 77.5716) (width 0.381) (layer "B.Cu") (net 4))
 (segment (start 96.5424 77.5716) (end 94.556 79.558) (width 0.381) (layer "B.Cu") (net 4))
 (segment (start 99.2124 77.498) (end 99.1388 77.5716) (width 0.381) (layer "B.Cu") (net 4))
 (segment (start 102.2096 83.2104) (end 100.4088 81.4096) (width 0.381) (layer "B.Cu") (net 4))
 (segment (start 100.4088 81.4096) (end 97.4852 81.4096) (width 0.381) (layer "B.Cu") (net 4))
 (segment (start 97.4852 81.4096) (end 95.6336 79.558) (width 0.381) (layer "B.Cu") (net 4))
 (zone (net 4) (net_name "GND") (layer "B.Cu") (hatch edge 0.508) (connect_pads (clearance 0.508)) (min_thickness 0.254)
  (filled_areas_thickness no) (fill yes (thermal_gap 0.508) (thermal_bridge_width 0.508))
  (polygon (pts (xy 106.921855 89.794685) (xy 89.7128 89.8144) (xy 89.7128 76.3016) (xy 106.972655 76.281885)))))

